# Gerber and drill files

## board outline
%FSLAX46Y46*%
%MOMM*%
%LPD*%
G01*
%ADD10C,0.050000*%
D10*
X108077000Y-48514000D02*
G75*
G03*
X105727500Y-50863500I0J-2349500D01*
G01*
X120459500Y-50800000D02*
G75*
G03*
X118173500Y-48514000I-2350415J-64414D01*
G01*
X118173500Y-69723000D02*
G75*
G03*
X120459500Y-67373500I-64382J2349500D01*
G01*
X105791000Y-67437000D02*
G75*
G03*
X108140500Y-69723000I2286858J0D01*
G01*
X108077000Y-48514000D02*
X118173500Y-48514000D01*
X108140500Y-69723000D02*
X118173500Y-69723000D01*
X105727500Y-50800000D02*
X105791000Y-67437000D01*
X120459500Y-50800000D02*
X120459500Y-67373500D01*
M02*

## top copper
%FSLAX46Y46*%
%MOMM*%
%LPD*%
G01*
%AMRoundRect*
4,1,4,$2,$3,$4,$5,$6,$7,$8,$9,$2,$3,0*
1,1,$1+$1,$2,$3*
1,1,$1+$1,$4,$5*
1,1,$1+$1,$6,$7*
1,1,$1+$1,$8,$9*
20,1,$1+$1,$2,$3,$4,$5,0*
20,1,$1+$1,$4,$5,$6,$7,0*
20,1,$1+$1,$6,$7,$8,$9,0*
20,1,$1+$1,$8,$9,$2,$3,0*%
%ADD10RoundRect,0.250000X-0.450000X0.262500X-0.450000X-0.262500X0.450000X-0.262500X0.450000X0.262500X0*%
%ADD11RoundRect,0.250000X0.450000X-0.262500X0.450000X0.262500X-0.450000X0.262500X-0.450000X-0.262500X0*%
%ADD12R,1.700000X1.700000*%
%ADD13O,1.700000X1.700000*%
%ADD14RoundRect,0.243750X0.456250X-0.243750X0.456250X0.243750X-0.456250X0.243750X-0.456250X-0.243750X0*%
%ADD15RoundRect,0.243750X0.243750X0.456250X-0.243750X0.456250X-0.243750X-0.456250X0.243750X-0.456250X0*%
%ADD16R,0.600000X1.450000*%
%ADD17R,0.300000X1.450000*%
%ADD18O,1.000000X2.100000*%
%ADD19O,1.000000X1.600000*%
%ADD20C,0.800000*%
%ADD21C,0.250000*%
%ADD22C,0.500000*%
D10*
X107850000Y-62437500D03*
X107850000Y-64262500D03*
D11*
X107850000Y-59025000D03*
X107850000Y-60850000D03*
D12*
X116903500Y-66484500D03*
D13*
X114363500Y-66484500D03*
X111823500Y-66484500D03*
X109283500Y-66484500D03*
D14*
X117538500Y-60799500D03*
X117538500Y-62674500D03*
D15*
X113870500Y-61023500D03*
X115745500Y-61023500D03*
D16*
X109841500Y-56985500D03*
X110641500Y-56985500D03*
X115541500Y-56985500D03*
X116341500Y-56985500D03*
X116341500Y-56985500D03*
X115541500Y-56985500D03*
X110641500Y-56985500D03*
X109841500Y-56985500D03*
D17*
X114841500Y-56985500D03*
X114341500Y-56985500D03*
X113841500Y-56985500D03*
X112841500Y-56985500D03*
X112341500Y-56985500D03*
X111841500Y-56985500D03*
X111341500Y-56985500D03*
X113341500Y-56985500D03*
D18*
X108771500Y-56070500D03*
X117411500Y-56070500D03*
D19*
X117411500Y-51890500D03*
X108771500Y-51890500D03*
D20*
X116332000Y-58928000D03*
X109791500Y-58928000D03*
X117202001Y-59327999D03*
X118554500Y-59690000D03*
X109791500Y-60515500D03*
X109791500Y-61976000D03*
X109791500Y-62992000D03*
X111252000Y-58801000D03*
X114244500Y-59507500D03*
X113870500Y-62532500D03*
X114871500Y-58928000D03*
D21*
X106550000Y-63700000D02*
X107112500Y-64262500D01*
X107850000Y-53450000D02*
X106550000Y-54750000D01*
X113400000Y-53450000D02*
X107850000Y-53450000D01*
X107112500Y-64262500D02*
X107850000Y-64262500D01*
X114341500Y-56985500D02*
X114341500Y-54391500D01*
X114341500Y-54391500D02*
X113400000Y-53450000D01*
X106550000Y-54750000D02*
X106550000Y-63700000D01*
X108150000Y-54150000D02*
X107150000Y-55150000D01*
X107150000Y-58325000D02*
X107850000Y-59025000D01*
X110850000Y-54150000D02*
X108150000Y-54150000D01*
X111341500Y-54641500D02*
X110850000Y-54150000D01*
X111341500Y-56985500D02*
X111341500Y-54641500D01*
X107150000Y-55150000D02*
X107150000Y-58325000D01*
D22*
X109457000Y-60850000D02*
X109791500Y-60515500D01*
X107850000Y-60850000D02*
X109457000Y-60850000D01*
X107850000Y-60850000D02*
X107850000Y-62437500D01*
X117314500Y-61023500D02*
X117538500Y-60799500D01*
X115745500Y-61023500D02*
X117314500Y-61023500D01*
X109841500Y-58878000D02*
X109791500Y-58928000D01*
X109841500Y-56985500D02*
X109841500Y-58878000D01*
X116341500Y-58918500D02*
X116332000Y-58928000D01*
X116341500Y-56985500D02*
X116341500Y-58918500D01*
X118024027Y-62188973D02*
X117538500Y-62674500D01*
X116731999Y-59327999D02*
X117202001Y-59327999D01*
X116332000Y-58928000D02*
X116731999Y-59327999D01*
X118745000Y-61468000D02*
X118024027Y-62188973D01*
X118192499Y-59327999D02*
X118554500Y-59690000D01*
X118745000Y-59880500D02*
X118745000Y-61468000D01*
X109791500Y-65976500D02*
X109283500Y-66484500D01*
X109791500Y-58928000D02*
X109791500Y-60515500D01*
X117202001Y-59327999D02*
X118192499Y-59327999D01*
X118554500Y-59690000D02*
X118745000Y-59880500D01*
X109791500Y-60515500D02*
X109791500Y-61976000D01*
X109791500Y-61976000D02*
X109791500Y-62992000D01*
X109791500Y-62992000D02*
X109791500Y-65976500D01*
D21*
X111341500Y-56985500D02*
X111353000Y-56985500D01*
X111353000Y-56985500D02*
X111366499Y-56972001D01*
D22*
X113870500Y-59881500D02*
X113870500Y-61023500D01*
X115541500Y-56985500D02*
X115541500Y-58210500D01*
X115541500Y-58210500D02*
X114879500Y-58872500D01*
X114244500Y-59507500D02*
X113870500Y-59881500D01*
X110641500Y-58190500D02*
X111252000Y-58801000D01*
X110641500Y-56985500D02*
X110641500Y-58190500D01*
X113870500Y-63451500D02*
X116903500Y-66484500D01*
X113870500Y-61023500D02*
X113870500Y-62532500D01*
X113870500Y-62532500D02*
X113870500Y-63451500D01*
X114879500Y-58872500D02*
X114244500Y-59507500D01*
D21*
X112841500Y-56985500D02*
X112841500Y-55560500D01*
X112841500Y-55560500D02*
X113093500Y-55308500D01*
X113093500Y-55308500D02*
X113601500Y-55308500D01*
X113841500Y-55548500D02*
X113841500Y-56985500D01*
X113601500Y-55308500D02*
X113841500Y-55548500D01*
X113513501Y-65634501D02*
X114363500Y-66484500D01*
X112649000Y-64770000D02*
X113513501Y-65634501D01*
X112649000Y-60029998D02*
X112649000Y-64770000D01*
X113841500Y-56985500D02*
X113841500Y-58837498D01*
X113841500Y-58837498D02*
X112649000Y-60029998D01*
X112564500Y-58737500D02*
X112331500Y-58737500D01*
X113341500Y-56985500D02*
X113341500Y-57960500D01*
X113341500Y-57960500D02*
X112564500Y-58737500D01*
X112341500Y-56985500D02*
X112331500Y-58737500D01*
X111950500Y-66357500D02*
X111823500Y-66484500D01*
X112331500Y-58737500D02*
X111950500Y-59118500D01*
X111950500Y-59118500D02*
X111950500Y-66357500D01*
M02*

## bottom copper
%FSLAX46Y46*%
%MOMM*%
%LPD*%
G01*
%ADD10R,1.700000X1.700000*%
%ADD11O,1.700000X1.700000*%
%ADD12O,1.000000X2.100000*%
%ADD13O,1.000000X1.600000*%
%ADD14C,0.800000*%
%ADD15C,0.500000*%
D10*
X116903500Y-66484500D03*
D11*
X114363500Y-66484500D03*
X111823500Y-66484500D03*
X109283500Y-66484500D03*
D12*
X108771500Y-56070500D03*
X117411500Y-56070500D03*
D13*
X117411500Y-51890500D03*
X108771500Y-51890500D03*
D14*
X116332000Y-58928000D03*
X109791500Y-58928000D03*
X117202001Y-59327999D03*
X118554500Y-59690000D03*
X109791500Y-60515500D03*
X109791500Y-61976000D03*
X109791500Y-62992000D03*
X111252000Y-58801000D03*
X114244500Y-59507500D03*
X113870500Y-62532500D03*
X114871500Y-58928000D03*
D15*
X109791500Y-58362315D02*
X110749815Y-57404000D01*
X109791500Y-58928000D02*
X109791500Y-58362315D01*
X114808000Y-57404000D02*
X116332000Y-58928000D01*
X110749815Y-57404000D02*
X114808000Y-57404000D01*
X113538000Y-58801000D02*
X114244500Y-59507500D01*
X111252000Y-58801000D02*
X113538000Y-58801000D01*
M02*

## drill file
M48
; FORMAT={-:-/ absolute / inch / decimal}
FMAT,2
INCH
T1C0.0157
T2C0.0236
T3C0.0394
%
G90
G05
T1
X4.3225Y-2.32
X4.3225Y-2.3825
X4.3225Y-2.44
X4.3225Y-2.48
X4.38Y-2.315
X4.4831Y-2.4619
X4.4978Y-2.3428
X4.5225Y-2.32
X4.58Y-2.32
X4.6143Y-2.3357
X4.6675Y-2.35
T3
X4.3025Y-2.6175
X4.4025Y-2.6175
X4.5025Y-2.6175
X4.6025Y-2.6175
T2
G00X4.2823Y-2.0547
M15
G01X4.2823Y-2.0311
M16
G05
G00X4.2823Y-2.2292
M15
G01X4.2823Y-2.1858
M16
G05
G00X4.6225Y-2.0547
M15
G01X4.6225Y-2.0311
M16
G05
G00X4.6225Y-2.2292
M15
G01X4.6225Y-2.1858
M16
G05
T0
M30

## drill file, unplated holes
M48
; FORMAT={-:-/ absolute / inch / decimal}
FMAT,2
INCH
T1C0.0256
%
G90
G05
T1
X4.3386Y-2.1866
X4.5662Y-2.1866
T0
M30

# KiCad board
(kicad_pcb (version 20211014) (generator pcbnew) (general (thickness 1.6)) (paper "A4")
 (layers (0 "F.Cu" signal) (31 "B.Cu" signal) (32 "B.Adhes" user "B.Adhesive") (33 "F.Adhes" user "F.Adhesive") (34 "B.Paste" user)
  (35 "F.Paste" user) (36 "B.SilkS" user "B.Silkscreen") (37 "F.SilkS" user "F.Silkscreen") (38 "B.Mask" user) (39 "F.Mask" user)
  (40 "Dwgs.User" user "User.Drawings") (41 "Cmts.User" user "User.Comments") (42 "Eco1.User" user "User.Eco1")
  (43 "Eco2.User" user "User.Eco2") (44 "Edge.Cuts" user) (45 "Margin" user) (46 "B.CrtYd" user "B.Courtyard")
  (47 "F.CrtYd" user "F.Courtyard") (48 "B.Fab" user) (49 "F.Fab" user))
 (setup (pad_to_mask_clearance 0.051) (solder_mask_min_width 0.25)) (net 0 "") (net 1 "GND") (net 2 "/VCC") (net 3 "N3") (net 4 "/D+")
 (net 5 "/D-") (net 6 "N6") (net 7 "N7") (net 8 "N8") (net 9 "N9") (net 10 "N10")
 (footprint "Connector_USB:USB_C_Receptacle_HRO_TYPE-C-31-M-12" (layer "F.Cu") (at 113.0915 52.9405 180)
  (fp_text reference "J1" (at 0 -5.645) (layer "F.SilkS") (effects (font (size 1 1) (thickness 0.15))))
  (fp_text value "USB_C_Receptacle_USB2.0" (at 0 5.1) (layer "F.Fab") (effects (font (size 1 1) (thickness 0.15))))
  (pad "" np_thru_hole circle locked (at 2.89 -2.6 180) (size 0.65 0.65) (drill 0.65) (layers *.Cu *.Mask))
  (pad "" np_thru_hole circle locked (at -2.89 -2.6 180) (size 0.65 0.65) (drill 0.65) (layers *.Cu *.Mask))
  (pad "A1" smd rect locked (at -3.25 -4.045 180) (size 0.6 1.45) (layers "F.Cu" "F.Paste" "F.Mask") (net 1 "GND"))
  (pad "A4" smd rect locked (at -2.45 -4.045 180) (size 0.6 1.45) (layers "F.Cu" "F.Paste" "F.Mask") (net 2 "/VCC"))
  (pad "A5" smd rect locked (at -1.25 -4.045 180) (size 0.3 1.45) (layers "F.Cu" "F.Paste" "F.Mask") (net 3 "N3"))
  (pad "A6" smd rect locked (at -0.25 -4.045 180) (size 0.3 1.45) (layers "F.Cu" "F.Paste" "F.Mask") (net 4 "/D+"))
  (pad "A7" smd rect locked (at 0.25 -4.045 180) (size 0.3 1.45) (layers "F.Cu" "F.Paste" "F.Mask") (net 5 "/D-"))
  (pad "A8" smd rect locked (at 1.25 -4.045 180) (size 0.3 1.45) (layers "F.Cu" "F.Paste" "F.Mask") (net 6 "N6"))
  (pad "A9" smd rect locked (at 2.45 -4.045 180) (size 0.6 1.45) (layers "F.Cu" "F.Paste" "F.Mask") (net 2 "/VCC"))
  (pad "A12" smd rect locked (at 3.25 -4.045 180) (size 0.6 1.45) (layers "F.Cu" "F.Paste" "F.Mask") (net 1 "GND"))
  (pad "B1" smd rect locked (at 3.25 -4.045 180) (size 0.6 1.45) (layers "F.Cu" "F.Paste" "F.Mask") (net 1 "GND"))
  (pad "B4" smd rect locked (at 2.45 -4.045 180) (size 0.6 1.45) (layers "F.Cu" "F.Paste" "F.Mask") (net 2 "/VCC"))
  (pad "B5" smd rect locked (at 1.75 -4.045 180) (size 0.3 1.45) (layers "F.Cu" "F.Paste" "F.Mask") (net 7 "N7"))
  (pad "B6" smd rect locked (at 0.75 -4.045 180) (size 0.3 1.45) (layers "F.Cu" "F.Paste" "F.Mask") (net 4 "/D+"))
  (pad "B7" smd rect locked (at -0.75 -4.045 180) (size 0.3 1.45) (layers "F.Cu" "F.Paste" "F.Mask") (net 5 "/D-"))
  (pad "B8" smd rect locked (at -1.75 -4.045 180) (size 0.3 1.45) (layers "F.Cu" "F.Paste" "F.Mask") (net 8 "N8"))
  (pad "B9" smd rect locked (at -2.45 -4.045 180) (size 0.6 1.45) (layers "F.Cu" "F.Paste" "F.Mask") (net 2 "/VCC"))
  (pad "B12" smd rect locked (at -3.25 -4.045 180) (size 0.6 1.45) (layers "F.Cu" "F.Paste" "F.Mask") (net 1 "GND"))
  (pad "S1" thru_hole oval locked (at -4.32 -3.13 180) (size 1 2.1) (drill oval 0.6 1.7) (layers *.Cu *.Mask) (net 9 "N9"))
  (pad "S1" thru_hole oval locked (at 4.32 1.05 180) (size 1 1.6) (drill oval 0.6 1.2) (layers *.Cu *.Mask) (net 9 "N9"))
  (pad "S1" thru_hole oval locked (at 4.32 -3.13 180) (size 1 2.1) (drill oval 0.6 1.7) (layers *.Cu *.Mask) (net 9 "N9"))
  (pad "S1" thru_hole oval locked (at -4.32 1.05 180) (size 1 1.6) (drill oval 0.6 1.2) (layers *.Cu *.Mask) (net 9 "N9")))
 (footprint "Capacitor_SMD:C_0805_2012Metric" (layer "F.Cu") (at 114.808 61.0235 180)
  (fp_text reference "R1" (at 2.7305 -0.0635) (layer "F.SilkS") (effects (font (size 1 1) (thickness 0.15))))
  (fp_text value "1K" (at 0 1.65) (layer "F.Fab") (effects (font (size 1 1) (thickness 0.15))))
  (pad "1" smd roundrect locked (at -0.9375 0 180) (size 0.975 1.4) (layers "F.Cu" "F.Paste" "F.Mask") (roundrect_rratio 0.25)
   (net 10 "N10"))
  (pad "2" smd roundrect locked (at 0.9375 0 180) (size 0.975 1.4) (layers "F.Cu" "F.Paste" "F.Mask") (roundrect_rratio 0.25) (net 2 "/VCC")))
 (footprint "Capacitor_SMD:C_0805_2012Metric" (layer "F.Cu") (at 117.5385 61.737 90)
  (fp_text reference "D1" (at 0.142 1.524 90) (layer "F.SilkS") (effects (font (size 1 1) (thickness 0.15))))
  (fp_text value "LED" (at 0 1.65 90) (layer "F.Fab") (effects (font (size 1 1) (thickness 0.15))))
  (pad "1" smd roundrect locked (at -0.9375 0 90) (size 0.975 1.4) (layers "F.Cu" "F.Paste" "F.Mask") (roundrect_rratio 0.25) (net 1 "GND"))
  (pad "2" smd roundrect locked (at 0.9375 0 90) (size 0.975 1.4) (layers "F.Cu" "F.Paste" "F.Mask") (roundrect_rratio 0.25) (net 10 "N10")))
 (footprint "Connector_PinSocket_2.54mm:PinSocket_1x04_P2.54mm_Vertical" (layer "F.Cu") (at 116.9035 66.4845 -90)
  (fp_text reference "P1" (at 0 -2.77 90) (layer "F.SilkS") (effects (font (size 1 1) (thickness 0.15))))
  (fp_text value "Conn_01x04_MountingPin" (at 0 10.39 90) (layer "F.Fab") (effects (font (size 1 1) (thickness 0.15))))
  (pad "1" thru_hole rect locked (at 0 0 270) (size 1.7 1.7) (drill 1) (layers *.Cu *.Mask) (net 2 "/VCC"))
  (pad "2" thru_hole oval locked (at 0 2.54 270) (size 1.7 1.7) (drill 1) (layers *.Cu *.Mask) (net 5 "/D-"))
  (pad "3" thru_hole oval locked (at 0 5.08 270) (size 1.7 1.7) (drill 1) (layers *.Cu *.Mask) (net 4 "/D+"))
  (pad "4" thru_hole oval locked (at 0 7.62 270) (size 1.7 1.7) (drill 1) (layers *.Cu *.Mask) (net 1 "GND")))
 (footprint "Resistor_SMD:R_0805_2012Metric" (layer "F.Cu") (at 107.85 63.35 -90)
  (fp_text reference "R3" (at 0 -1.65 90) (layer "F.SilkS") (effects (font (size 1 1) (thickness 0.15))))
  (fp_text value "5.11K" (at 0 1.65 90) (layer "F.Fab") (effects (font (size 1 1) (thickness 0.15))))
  (pad "1" smd roundrect locked (at -0.9125 0 270) (size 1.025 1.4) (layers "F.Cu" "F.Paste" "F.Mask") (roundrect_rratio 0.243902439)
   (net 1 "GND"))
  (pad "2" smd roundrect locked (at 0.9125 0 270) (size 1.025 1.4) (layers "F.Cu" "F.Paste" "F.Mask") (roundrect_rratio 0.243902439)
   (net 3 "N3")))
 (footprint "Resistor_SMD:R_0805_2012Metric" (layer "F.Cu") (at 107.85 59.9375 90)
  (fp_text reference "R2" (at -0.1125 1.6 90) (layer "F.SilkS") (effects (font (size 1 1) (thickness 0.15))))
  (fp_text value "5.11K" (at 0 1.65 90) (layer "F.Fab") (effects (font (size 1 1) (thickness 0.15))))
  (pad "1" smd roundrect locked (at -0.9125 0 90) (size 1.025 1.4) (layers "F.Cu" "F.Paste" "F.Mask") (roundrect_rratio 0.243902439)
   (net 1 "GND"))
  (pad "2" smd roundrect locked (at 0.9125 0 90) (size 1.025 1.4) (layers "F.Cu" "F.Paste" "F.Mask") (roundrect_rratio 0.243902439)
   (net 7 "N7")))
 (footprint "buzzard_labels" (layer "B.Cu") (at 113.2 58.5 180)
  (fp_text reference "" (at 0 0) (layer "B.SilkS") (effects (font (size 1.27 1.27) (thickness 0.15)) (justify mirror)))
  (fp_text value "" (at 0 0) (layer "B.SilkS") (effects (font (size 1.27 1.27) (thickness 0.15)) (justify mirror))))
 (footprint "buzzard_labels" (layer "B.Cu") (at 114.45 59.8 180)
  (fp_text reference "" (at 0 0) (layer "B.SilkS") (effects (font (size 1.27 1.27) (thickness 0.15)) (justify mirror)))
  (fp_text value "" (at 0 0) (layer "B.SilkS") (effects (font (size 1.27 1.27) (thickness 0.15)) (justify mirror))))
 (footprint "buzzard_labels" (layer "B.Cu") (at 116.1 61.1 180)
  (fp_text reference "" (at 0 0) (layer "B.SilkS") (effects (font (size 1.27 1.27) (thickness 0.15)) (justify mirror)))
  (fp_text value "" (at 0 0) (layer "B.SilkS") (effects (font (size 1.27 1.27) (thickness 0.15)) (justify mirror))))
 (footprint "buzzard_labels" (layer "B.Cu") (at 113.25 64.25 180)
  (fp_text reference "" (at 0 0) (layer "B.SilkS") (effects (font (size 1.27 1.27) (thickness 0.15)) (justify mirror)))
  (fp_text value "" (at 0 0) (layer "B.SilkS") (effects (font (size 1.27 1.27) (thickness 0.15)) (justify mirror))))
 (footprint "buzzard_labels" (layer "B.Cu") (at 113.05 49.8 180)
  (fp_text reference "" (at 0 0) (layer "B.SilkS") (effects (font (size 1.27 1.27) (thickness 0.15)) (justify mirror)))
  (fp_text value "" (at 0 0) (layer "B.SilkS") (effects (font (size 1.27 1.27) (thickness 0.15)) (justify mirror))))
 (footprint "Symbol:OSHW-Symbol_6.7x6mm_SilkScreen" (layer "B.Cu") (at 113.1 54.05 180)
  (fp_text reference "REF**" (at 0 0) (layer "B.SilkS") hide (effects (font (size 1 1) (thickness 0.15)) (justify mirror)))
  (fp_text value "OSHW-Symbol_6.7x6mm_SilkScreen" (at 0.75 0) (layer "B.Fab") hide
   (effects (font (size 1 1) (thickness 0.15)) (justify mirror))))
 (gr_arc (start 108.1405 69.723) (mid 106.483106 69.076051) (end 105.791 67.437) (layer "Edge.Cuts") (width 0.05))
 (gr_line (start 120.4595 50.8) (end 120.4595 67.3735) (layer "Edge.Cuts") (width 0.05))
 (gr_line (start 105.7275 50.8) (end 105.791 67.437) (layer "Edge.Cuts") (width 0.05))
 (gr_arc (start 105.7275 50.8635) (mid 106.415653 49.202153) (end 108.077 48.514) (layer "Edge.Cuts") (width 0.05))
 (gr_line (start 108.1405 69.723) (end 118.1735 69.723) (layer "Edge.Cuts") (width 0.05))
 (gr_line (start 108.077 48.514) (end 118.1735 48.514) (layer "Edge.Cuts") (width 0.05))
 (gr_arc (start 120.4595 67.3735) (mid 119.793698 69.012551) (end 118.1735 69.723) (layer "Edge.Cuts") (width 0.05))
 (gr_arc (start 118.1735 48.514) (mid 119.771703 49.201797) (end 120.4595 50.8) (layer "Edge.Cuts") (width 0.05))
 (segment (start 115.7455 61.0235) (end 117.3145 61.0235) (width 0.5) (layer "F.Cu") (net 10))
 (segment (start 117.3145 61.0235) (end 117.5385 60.7995) (width 0.5) (layer "F.Cu") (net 10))
 (segment (start 117.202001 59.327999) (end 118.192499 59.327999) (width 0.5) (layer "F.Cu") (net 1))
 (segment (start 118.5545 59.69) (end 118.745 59.8805) (width 0.5) (layer "F.Cu") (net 1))
 (segment (start 109.7915 60.5155) (end 109.7915 61.976) (width 0.5) (layer "F.Cu") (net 1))
 (segment (start 109.7915 61.976) (end 109.7915 62.992) (width 0.5) (layer "F.Cu") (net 1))
 (segment (start 109.7915 62.992) (end 109.7915 65.9765) (width 0.5) (layer "F.Cu") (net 1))
 (segment (start 118.192499 59.327999) (end 118.5545 59.69) (width 0.5) (layer "F.Cu") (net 1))
 (segment (start 107.85 60.85) (end 109.457 60.85) (width 0.5) (layer "F.Cu") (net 1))
 (segment (start 116.731999 59.327999) (end 117.202001 59.327999) (width 0.5) (layer "F.Cu") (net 1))
 (segment (start 109.7915 65.9765) (end 109.2835 66.4845) (width 0.5) (layer "F.Cu") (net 1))
 (segment (start 107.85 60.85) (end 107.85 62.4375) (width 0.5) (layer "F.Cu") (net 1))
 (segment (start 118.024027 62.188973) (end 117.5385 62.6745) (width 0.5) (layer "F.Cu") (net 1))
 (segment (start 116.3415 58.9185) (end 116.332 58.928) (width 0.5) (layer "F.Cu") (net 1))
 (segment (start 109.7915 58.928) (end 109.7915 60.5155) (width 0.5) (layer "F.Cu") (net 1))
 (segment (start 116.332 58.928) (end 116.731999 59.327999) (width 0.5) (layer "F.Cu") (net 1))
 (segment (start 109.8415 56.9855) (end 109.8415 58.878) (width 0.5) (layer "F.Cu") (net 1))
 (segment (start 116.3415 56.9855) (end 116.3415 58.9185) (width 0.5) (layer "F.Cu") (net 1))
 (segment (start 118.745 61.468) (end 118.024027 62.188973) (width 0.5) (layer "F.Cu") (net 1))
 (segment (start 109.8415 58.878) (end 109.7915 58.928) (width 0.5) (layer "F.Cu") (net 1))
 (segment (start 118.745 59.8805) (end 118.745 61.468) (width 0.5) (layer "F.Cu") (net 1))
 (segment (start 109.457 60.85) (end 109.7915 60.5155) (width 0.5) (layer "F.Cu") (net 1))
 (via (at 109.7915 60.5155) (size 0.8) (drill 0.4) (layers "F.Cu" "B.Cu") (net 1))
 (via (at 117.202001 59.327999) (size 0.8) (drill 0.4) (layers "F.Cu" "B.Cu") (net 1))
 (via (at 118.5545 59.69) (size 0.8) (drill 0.4) (layers "F.Cu" "B.Cu") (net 1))
 (via (at 109.7915 58.928) (size 0.8) (drill 0.4) (layers "F.Cu" "B.Cu") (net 1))
 (via (at 109.7915 62.992) (size 0.8) (drill 0.4) (layers "F.Cu" "B.Cu") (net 1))
 (via (at 109.7915 61.976) (size 0.8) (drill 0.4) (layers "F.Cu" "B.Cu") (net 1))
 (via (at 116.332 58.928) (size 0.8) (drill 0.4) (layers "F.Cu" "B.Cu") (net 1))
 (segment (start 109.7915 58.928) (end 109.7915 58.362315) (width 0.5) (layer "B.Cu") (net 1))
 (segment (start 110.749815 57.404) (end 114.808 57.404) (width 0.5) (layer "B.Cu") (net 1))
 (segment (start 114.808 57.404) (end 116.332 58.928) (width 0.5) (layer "B.Cu") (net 1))
 (segment (start 109.7915 58.362315) (end 110.749815 57.404) (width 0.5) (layer "B.Cu") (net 1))
 (segment (start 107.85 53.45) (end 106.55 54.75) (width 0.25) (layer "F.Cu") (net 3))
 (segment (start 113.4 53.45) (end 107.85 53.45) (width 0.25) (layer "F.Cu") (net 3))
 (segment (start 107.1125 64.2625) (end 107.85 64.2625) (width 0.25) (layer "F.Cu") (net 3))
 (segment (start 106.55 63.7) (end 107.1125 64.2625) (width 0.25) (layer "F.Cu") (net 3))
 (segment (start 114.3415 54.3915) (end 113.4 53.45) (width 0.25) (layer "F.Cu") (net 3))
 (segment (start 114.3415 56.9855) (end 114.3415 54.3915) (width 0.25) (layer "F.Cu") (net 3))
 (segment (start 106.55 54.75) (end 106.55 63.7) (width 0.25) (layer "F.Cu") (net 3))
 (segment (start 108.15 54.15) (end 107.15 55.15) (width 0.25) (layer "F.Cu") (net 7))
 (segment (start 107.15 55.15) (end 107.15 58.325) (width 0.25) (layer "F.Cu") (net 7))
 (segment (start 107.15 58.325) (end 107.85 59.025) (width 0.25) (layer "F.Cu") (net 7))
 (segment (start 111.3415 56.9855) (end 111.353 56.9855) (width 0.25) (layer "F.Cu") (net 7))
 (segment (start 111.353 56.9855) (end 111.366499 56.972001) (width 0.25) (layer "F.Cu") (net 7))
 (segment (start 111.3415 54.6415) (end 110.85 54.15) (width 0.25) (layer "F.Cu") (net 7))
 (segment (start 111.3415 56.9855) (end 111.3415 54.6415) (width 0.25) (layer "F.Cu") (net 7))
 (segment (start 110.85 54.15) (end 108.15 54.15) (width 0.25) (layer "F.Cu") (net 7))
 (segment (start 114.2445 59.5075) (end 113.8705 59.8815) (width 0.5) (layer "F.Cu") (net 2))
 (segment (start 113.8705 62.5325) (end 113.8705 63.4515) (width 0.5) (layer "F.Cu") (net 2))
 (segment (start 114.8795 58.8725) (end 114.2445 59.5075) (width 0.5) (layer "F.Cu") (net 2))
 (segment (start 115.5415 56.9855) (end 115.5415 58.2105) (width 0.5) (layer "F.Cu") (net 2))
 (segment (start 113.8705 59.8815) (end 113.8705 61.0235) (width 0.5) (layer "F.Cu") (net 2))
 (segment (start 113.8705 63.4515) (end 116.9035 66.4845) (width 0.5) (layer "F.Cu") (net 2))
 (segment (start 110.6415 56.9855) (end 110.6415 58.1905) (width 0.5) (layer "F.Cu") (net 2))
 (segment (start 113.8705 61.0235) (end 113.8705 62.5325) (width 0.5) (layer "F.Cu") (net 2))
 (segment (start 115.5415 58.2105) (end 114.8795 58.8725) (width 0.5) (layer "F.Cu") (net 2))
 (segment (start 110.6415 58.1905) (end 111.252 58.801) (width 0.5) (layer "F.Cu") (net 2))
 (via (at 113.8705 62.5325) (size 0.8) (drill 0.4) (layers "F.Cu" "B.Cu") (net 2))
 (via (at 114.8715 58.928) (size 0.8) (drill 0.4) (layers "F.Cu" "B.Cu") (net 2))
 (via (at 114.2445 59.5075) (size 0.8) (drill 0.4) (layers "F.Cu" "B.Cu") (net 2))
 (via (at 111.252 58.801) (size 0.8) (drill 0.4) (layers "F.Cu" "B.Cu") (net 2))
 (segment (start 113.538 58.801) (end 114.2445 59.5075) (width 0.5) (layer "B.Cu") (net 2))
 (segment (start 111.252 58.801) (end 113.538 58.801) (width 0.5) (layer "B.Cu") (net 2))
 (segment (start 113.6015 55.3085) (end 113.8415 55.5485) (width 0.25) (layer "F.Cu") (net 5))
 (segment (start 113.8415 56.9855) (end 113.8415 58.837498) (width 0.25) (layer "F.Cu") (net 5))
 (segment (start 112.8415 55.5605) (end 113.0935 55.3085) (width 0.25) (layer "F.Cu") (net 5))
 (segment (start 112.649 60.029998) (end 112.649 64.77) (width 0.25) (layer "F.Cu") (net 5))
 (segment (start 112.649 64.77) (end 113.513501 65.634501) (width 0.25) (layer "F.Cu") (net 5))
 (segment (start 113.513501 65.634501) (end 114.3635 66.4845) (width 0.25) (layer "F.Cu") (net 5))
 (segment (start 113.8415 55.5485) (end 113.8415 56.9855) (width 0.25) (layer "F.Cu") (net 5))
 (segment (start 113.8415 58.837498) (end 112.649 60.029998) (width 0.25) (layer "F.Cu") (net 5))
 (segment (start 113.0935 55.3085) (end 113.6015 55.3085) (width 0.25) (layer "F.Cu") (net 5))
 (segment (start 112.8415 56.9855) (end 112.8415 55.5605) (width 0.25) (layer "F.Cu") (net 5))
 (segment (start 111.9505 66.3575) (end 111.8235 66.4845) (width 0.25) (layer "F.Cu") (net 4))
 (segment (start 112.3315 58.7375) (end 111.9505 59.1185) (width 0.25) (layer "F.Cu") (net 4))
 (segment (start 112.3415 56.9855) (end 112.3315 58.7375) (width 0.25) (layer "F.Cu") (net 4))
 (segment (start 112.5645 58.7375) (end 112.3315 58.7375) (width 0.25) (layer "F.Cu") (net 4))
 (segment (start 113.3415 57.9605) (end 112.5645 58.7375) (width 0.25) (layer "F.Cu") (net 4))
 (segment (start 113.3415 56.9855) (end 113.3415 57.9605) (width 0.25) (layer "F.Cu") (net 4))
 (segment (start 111.9505 59.1185) (end 111.9505 66.3575) (width 0.25) (layer "F.Cu") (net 4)))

